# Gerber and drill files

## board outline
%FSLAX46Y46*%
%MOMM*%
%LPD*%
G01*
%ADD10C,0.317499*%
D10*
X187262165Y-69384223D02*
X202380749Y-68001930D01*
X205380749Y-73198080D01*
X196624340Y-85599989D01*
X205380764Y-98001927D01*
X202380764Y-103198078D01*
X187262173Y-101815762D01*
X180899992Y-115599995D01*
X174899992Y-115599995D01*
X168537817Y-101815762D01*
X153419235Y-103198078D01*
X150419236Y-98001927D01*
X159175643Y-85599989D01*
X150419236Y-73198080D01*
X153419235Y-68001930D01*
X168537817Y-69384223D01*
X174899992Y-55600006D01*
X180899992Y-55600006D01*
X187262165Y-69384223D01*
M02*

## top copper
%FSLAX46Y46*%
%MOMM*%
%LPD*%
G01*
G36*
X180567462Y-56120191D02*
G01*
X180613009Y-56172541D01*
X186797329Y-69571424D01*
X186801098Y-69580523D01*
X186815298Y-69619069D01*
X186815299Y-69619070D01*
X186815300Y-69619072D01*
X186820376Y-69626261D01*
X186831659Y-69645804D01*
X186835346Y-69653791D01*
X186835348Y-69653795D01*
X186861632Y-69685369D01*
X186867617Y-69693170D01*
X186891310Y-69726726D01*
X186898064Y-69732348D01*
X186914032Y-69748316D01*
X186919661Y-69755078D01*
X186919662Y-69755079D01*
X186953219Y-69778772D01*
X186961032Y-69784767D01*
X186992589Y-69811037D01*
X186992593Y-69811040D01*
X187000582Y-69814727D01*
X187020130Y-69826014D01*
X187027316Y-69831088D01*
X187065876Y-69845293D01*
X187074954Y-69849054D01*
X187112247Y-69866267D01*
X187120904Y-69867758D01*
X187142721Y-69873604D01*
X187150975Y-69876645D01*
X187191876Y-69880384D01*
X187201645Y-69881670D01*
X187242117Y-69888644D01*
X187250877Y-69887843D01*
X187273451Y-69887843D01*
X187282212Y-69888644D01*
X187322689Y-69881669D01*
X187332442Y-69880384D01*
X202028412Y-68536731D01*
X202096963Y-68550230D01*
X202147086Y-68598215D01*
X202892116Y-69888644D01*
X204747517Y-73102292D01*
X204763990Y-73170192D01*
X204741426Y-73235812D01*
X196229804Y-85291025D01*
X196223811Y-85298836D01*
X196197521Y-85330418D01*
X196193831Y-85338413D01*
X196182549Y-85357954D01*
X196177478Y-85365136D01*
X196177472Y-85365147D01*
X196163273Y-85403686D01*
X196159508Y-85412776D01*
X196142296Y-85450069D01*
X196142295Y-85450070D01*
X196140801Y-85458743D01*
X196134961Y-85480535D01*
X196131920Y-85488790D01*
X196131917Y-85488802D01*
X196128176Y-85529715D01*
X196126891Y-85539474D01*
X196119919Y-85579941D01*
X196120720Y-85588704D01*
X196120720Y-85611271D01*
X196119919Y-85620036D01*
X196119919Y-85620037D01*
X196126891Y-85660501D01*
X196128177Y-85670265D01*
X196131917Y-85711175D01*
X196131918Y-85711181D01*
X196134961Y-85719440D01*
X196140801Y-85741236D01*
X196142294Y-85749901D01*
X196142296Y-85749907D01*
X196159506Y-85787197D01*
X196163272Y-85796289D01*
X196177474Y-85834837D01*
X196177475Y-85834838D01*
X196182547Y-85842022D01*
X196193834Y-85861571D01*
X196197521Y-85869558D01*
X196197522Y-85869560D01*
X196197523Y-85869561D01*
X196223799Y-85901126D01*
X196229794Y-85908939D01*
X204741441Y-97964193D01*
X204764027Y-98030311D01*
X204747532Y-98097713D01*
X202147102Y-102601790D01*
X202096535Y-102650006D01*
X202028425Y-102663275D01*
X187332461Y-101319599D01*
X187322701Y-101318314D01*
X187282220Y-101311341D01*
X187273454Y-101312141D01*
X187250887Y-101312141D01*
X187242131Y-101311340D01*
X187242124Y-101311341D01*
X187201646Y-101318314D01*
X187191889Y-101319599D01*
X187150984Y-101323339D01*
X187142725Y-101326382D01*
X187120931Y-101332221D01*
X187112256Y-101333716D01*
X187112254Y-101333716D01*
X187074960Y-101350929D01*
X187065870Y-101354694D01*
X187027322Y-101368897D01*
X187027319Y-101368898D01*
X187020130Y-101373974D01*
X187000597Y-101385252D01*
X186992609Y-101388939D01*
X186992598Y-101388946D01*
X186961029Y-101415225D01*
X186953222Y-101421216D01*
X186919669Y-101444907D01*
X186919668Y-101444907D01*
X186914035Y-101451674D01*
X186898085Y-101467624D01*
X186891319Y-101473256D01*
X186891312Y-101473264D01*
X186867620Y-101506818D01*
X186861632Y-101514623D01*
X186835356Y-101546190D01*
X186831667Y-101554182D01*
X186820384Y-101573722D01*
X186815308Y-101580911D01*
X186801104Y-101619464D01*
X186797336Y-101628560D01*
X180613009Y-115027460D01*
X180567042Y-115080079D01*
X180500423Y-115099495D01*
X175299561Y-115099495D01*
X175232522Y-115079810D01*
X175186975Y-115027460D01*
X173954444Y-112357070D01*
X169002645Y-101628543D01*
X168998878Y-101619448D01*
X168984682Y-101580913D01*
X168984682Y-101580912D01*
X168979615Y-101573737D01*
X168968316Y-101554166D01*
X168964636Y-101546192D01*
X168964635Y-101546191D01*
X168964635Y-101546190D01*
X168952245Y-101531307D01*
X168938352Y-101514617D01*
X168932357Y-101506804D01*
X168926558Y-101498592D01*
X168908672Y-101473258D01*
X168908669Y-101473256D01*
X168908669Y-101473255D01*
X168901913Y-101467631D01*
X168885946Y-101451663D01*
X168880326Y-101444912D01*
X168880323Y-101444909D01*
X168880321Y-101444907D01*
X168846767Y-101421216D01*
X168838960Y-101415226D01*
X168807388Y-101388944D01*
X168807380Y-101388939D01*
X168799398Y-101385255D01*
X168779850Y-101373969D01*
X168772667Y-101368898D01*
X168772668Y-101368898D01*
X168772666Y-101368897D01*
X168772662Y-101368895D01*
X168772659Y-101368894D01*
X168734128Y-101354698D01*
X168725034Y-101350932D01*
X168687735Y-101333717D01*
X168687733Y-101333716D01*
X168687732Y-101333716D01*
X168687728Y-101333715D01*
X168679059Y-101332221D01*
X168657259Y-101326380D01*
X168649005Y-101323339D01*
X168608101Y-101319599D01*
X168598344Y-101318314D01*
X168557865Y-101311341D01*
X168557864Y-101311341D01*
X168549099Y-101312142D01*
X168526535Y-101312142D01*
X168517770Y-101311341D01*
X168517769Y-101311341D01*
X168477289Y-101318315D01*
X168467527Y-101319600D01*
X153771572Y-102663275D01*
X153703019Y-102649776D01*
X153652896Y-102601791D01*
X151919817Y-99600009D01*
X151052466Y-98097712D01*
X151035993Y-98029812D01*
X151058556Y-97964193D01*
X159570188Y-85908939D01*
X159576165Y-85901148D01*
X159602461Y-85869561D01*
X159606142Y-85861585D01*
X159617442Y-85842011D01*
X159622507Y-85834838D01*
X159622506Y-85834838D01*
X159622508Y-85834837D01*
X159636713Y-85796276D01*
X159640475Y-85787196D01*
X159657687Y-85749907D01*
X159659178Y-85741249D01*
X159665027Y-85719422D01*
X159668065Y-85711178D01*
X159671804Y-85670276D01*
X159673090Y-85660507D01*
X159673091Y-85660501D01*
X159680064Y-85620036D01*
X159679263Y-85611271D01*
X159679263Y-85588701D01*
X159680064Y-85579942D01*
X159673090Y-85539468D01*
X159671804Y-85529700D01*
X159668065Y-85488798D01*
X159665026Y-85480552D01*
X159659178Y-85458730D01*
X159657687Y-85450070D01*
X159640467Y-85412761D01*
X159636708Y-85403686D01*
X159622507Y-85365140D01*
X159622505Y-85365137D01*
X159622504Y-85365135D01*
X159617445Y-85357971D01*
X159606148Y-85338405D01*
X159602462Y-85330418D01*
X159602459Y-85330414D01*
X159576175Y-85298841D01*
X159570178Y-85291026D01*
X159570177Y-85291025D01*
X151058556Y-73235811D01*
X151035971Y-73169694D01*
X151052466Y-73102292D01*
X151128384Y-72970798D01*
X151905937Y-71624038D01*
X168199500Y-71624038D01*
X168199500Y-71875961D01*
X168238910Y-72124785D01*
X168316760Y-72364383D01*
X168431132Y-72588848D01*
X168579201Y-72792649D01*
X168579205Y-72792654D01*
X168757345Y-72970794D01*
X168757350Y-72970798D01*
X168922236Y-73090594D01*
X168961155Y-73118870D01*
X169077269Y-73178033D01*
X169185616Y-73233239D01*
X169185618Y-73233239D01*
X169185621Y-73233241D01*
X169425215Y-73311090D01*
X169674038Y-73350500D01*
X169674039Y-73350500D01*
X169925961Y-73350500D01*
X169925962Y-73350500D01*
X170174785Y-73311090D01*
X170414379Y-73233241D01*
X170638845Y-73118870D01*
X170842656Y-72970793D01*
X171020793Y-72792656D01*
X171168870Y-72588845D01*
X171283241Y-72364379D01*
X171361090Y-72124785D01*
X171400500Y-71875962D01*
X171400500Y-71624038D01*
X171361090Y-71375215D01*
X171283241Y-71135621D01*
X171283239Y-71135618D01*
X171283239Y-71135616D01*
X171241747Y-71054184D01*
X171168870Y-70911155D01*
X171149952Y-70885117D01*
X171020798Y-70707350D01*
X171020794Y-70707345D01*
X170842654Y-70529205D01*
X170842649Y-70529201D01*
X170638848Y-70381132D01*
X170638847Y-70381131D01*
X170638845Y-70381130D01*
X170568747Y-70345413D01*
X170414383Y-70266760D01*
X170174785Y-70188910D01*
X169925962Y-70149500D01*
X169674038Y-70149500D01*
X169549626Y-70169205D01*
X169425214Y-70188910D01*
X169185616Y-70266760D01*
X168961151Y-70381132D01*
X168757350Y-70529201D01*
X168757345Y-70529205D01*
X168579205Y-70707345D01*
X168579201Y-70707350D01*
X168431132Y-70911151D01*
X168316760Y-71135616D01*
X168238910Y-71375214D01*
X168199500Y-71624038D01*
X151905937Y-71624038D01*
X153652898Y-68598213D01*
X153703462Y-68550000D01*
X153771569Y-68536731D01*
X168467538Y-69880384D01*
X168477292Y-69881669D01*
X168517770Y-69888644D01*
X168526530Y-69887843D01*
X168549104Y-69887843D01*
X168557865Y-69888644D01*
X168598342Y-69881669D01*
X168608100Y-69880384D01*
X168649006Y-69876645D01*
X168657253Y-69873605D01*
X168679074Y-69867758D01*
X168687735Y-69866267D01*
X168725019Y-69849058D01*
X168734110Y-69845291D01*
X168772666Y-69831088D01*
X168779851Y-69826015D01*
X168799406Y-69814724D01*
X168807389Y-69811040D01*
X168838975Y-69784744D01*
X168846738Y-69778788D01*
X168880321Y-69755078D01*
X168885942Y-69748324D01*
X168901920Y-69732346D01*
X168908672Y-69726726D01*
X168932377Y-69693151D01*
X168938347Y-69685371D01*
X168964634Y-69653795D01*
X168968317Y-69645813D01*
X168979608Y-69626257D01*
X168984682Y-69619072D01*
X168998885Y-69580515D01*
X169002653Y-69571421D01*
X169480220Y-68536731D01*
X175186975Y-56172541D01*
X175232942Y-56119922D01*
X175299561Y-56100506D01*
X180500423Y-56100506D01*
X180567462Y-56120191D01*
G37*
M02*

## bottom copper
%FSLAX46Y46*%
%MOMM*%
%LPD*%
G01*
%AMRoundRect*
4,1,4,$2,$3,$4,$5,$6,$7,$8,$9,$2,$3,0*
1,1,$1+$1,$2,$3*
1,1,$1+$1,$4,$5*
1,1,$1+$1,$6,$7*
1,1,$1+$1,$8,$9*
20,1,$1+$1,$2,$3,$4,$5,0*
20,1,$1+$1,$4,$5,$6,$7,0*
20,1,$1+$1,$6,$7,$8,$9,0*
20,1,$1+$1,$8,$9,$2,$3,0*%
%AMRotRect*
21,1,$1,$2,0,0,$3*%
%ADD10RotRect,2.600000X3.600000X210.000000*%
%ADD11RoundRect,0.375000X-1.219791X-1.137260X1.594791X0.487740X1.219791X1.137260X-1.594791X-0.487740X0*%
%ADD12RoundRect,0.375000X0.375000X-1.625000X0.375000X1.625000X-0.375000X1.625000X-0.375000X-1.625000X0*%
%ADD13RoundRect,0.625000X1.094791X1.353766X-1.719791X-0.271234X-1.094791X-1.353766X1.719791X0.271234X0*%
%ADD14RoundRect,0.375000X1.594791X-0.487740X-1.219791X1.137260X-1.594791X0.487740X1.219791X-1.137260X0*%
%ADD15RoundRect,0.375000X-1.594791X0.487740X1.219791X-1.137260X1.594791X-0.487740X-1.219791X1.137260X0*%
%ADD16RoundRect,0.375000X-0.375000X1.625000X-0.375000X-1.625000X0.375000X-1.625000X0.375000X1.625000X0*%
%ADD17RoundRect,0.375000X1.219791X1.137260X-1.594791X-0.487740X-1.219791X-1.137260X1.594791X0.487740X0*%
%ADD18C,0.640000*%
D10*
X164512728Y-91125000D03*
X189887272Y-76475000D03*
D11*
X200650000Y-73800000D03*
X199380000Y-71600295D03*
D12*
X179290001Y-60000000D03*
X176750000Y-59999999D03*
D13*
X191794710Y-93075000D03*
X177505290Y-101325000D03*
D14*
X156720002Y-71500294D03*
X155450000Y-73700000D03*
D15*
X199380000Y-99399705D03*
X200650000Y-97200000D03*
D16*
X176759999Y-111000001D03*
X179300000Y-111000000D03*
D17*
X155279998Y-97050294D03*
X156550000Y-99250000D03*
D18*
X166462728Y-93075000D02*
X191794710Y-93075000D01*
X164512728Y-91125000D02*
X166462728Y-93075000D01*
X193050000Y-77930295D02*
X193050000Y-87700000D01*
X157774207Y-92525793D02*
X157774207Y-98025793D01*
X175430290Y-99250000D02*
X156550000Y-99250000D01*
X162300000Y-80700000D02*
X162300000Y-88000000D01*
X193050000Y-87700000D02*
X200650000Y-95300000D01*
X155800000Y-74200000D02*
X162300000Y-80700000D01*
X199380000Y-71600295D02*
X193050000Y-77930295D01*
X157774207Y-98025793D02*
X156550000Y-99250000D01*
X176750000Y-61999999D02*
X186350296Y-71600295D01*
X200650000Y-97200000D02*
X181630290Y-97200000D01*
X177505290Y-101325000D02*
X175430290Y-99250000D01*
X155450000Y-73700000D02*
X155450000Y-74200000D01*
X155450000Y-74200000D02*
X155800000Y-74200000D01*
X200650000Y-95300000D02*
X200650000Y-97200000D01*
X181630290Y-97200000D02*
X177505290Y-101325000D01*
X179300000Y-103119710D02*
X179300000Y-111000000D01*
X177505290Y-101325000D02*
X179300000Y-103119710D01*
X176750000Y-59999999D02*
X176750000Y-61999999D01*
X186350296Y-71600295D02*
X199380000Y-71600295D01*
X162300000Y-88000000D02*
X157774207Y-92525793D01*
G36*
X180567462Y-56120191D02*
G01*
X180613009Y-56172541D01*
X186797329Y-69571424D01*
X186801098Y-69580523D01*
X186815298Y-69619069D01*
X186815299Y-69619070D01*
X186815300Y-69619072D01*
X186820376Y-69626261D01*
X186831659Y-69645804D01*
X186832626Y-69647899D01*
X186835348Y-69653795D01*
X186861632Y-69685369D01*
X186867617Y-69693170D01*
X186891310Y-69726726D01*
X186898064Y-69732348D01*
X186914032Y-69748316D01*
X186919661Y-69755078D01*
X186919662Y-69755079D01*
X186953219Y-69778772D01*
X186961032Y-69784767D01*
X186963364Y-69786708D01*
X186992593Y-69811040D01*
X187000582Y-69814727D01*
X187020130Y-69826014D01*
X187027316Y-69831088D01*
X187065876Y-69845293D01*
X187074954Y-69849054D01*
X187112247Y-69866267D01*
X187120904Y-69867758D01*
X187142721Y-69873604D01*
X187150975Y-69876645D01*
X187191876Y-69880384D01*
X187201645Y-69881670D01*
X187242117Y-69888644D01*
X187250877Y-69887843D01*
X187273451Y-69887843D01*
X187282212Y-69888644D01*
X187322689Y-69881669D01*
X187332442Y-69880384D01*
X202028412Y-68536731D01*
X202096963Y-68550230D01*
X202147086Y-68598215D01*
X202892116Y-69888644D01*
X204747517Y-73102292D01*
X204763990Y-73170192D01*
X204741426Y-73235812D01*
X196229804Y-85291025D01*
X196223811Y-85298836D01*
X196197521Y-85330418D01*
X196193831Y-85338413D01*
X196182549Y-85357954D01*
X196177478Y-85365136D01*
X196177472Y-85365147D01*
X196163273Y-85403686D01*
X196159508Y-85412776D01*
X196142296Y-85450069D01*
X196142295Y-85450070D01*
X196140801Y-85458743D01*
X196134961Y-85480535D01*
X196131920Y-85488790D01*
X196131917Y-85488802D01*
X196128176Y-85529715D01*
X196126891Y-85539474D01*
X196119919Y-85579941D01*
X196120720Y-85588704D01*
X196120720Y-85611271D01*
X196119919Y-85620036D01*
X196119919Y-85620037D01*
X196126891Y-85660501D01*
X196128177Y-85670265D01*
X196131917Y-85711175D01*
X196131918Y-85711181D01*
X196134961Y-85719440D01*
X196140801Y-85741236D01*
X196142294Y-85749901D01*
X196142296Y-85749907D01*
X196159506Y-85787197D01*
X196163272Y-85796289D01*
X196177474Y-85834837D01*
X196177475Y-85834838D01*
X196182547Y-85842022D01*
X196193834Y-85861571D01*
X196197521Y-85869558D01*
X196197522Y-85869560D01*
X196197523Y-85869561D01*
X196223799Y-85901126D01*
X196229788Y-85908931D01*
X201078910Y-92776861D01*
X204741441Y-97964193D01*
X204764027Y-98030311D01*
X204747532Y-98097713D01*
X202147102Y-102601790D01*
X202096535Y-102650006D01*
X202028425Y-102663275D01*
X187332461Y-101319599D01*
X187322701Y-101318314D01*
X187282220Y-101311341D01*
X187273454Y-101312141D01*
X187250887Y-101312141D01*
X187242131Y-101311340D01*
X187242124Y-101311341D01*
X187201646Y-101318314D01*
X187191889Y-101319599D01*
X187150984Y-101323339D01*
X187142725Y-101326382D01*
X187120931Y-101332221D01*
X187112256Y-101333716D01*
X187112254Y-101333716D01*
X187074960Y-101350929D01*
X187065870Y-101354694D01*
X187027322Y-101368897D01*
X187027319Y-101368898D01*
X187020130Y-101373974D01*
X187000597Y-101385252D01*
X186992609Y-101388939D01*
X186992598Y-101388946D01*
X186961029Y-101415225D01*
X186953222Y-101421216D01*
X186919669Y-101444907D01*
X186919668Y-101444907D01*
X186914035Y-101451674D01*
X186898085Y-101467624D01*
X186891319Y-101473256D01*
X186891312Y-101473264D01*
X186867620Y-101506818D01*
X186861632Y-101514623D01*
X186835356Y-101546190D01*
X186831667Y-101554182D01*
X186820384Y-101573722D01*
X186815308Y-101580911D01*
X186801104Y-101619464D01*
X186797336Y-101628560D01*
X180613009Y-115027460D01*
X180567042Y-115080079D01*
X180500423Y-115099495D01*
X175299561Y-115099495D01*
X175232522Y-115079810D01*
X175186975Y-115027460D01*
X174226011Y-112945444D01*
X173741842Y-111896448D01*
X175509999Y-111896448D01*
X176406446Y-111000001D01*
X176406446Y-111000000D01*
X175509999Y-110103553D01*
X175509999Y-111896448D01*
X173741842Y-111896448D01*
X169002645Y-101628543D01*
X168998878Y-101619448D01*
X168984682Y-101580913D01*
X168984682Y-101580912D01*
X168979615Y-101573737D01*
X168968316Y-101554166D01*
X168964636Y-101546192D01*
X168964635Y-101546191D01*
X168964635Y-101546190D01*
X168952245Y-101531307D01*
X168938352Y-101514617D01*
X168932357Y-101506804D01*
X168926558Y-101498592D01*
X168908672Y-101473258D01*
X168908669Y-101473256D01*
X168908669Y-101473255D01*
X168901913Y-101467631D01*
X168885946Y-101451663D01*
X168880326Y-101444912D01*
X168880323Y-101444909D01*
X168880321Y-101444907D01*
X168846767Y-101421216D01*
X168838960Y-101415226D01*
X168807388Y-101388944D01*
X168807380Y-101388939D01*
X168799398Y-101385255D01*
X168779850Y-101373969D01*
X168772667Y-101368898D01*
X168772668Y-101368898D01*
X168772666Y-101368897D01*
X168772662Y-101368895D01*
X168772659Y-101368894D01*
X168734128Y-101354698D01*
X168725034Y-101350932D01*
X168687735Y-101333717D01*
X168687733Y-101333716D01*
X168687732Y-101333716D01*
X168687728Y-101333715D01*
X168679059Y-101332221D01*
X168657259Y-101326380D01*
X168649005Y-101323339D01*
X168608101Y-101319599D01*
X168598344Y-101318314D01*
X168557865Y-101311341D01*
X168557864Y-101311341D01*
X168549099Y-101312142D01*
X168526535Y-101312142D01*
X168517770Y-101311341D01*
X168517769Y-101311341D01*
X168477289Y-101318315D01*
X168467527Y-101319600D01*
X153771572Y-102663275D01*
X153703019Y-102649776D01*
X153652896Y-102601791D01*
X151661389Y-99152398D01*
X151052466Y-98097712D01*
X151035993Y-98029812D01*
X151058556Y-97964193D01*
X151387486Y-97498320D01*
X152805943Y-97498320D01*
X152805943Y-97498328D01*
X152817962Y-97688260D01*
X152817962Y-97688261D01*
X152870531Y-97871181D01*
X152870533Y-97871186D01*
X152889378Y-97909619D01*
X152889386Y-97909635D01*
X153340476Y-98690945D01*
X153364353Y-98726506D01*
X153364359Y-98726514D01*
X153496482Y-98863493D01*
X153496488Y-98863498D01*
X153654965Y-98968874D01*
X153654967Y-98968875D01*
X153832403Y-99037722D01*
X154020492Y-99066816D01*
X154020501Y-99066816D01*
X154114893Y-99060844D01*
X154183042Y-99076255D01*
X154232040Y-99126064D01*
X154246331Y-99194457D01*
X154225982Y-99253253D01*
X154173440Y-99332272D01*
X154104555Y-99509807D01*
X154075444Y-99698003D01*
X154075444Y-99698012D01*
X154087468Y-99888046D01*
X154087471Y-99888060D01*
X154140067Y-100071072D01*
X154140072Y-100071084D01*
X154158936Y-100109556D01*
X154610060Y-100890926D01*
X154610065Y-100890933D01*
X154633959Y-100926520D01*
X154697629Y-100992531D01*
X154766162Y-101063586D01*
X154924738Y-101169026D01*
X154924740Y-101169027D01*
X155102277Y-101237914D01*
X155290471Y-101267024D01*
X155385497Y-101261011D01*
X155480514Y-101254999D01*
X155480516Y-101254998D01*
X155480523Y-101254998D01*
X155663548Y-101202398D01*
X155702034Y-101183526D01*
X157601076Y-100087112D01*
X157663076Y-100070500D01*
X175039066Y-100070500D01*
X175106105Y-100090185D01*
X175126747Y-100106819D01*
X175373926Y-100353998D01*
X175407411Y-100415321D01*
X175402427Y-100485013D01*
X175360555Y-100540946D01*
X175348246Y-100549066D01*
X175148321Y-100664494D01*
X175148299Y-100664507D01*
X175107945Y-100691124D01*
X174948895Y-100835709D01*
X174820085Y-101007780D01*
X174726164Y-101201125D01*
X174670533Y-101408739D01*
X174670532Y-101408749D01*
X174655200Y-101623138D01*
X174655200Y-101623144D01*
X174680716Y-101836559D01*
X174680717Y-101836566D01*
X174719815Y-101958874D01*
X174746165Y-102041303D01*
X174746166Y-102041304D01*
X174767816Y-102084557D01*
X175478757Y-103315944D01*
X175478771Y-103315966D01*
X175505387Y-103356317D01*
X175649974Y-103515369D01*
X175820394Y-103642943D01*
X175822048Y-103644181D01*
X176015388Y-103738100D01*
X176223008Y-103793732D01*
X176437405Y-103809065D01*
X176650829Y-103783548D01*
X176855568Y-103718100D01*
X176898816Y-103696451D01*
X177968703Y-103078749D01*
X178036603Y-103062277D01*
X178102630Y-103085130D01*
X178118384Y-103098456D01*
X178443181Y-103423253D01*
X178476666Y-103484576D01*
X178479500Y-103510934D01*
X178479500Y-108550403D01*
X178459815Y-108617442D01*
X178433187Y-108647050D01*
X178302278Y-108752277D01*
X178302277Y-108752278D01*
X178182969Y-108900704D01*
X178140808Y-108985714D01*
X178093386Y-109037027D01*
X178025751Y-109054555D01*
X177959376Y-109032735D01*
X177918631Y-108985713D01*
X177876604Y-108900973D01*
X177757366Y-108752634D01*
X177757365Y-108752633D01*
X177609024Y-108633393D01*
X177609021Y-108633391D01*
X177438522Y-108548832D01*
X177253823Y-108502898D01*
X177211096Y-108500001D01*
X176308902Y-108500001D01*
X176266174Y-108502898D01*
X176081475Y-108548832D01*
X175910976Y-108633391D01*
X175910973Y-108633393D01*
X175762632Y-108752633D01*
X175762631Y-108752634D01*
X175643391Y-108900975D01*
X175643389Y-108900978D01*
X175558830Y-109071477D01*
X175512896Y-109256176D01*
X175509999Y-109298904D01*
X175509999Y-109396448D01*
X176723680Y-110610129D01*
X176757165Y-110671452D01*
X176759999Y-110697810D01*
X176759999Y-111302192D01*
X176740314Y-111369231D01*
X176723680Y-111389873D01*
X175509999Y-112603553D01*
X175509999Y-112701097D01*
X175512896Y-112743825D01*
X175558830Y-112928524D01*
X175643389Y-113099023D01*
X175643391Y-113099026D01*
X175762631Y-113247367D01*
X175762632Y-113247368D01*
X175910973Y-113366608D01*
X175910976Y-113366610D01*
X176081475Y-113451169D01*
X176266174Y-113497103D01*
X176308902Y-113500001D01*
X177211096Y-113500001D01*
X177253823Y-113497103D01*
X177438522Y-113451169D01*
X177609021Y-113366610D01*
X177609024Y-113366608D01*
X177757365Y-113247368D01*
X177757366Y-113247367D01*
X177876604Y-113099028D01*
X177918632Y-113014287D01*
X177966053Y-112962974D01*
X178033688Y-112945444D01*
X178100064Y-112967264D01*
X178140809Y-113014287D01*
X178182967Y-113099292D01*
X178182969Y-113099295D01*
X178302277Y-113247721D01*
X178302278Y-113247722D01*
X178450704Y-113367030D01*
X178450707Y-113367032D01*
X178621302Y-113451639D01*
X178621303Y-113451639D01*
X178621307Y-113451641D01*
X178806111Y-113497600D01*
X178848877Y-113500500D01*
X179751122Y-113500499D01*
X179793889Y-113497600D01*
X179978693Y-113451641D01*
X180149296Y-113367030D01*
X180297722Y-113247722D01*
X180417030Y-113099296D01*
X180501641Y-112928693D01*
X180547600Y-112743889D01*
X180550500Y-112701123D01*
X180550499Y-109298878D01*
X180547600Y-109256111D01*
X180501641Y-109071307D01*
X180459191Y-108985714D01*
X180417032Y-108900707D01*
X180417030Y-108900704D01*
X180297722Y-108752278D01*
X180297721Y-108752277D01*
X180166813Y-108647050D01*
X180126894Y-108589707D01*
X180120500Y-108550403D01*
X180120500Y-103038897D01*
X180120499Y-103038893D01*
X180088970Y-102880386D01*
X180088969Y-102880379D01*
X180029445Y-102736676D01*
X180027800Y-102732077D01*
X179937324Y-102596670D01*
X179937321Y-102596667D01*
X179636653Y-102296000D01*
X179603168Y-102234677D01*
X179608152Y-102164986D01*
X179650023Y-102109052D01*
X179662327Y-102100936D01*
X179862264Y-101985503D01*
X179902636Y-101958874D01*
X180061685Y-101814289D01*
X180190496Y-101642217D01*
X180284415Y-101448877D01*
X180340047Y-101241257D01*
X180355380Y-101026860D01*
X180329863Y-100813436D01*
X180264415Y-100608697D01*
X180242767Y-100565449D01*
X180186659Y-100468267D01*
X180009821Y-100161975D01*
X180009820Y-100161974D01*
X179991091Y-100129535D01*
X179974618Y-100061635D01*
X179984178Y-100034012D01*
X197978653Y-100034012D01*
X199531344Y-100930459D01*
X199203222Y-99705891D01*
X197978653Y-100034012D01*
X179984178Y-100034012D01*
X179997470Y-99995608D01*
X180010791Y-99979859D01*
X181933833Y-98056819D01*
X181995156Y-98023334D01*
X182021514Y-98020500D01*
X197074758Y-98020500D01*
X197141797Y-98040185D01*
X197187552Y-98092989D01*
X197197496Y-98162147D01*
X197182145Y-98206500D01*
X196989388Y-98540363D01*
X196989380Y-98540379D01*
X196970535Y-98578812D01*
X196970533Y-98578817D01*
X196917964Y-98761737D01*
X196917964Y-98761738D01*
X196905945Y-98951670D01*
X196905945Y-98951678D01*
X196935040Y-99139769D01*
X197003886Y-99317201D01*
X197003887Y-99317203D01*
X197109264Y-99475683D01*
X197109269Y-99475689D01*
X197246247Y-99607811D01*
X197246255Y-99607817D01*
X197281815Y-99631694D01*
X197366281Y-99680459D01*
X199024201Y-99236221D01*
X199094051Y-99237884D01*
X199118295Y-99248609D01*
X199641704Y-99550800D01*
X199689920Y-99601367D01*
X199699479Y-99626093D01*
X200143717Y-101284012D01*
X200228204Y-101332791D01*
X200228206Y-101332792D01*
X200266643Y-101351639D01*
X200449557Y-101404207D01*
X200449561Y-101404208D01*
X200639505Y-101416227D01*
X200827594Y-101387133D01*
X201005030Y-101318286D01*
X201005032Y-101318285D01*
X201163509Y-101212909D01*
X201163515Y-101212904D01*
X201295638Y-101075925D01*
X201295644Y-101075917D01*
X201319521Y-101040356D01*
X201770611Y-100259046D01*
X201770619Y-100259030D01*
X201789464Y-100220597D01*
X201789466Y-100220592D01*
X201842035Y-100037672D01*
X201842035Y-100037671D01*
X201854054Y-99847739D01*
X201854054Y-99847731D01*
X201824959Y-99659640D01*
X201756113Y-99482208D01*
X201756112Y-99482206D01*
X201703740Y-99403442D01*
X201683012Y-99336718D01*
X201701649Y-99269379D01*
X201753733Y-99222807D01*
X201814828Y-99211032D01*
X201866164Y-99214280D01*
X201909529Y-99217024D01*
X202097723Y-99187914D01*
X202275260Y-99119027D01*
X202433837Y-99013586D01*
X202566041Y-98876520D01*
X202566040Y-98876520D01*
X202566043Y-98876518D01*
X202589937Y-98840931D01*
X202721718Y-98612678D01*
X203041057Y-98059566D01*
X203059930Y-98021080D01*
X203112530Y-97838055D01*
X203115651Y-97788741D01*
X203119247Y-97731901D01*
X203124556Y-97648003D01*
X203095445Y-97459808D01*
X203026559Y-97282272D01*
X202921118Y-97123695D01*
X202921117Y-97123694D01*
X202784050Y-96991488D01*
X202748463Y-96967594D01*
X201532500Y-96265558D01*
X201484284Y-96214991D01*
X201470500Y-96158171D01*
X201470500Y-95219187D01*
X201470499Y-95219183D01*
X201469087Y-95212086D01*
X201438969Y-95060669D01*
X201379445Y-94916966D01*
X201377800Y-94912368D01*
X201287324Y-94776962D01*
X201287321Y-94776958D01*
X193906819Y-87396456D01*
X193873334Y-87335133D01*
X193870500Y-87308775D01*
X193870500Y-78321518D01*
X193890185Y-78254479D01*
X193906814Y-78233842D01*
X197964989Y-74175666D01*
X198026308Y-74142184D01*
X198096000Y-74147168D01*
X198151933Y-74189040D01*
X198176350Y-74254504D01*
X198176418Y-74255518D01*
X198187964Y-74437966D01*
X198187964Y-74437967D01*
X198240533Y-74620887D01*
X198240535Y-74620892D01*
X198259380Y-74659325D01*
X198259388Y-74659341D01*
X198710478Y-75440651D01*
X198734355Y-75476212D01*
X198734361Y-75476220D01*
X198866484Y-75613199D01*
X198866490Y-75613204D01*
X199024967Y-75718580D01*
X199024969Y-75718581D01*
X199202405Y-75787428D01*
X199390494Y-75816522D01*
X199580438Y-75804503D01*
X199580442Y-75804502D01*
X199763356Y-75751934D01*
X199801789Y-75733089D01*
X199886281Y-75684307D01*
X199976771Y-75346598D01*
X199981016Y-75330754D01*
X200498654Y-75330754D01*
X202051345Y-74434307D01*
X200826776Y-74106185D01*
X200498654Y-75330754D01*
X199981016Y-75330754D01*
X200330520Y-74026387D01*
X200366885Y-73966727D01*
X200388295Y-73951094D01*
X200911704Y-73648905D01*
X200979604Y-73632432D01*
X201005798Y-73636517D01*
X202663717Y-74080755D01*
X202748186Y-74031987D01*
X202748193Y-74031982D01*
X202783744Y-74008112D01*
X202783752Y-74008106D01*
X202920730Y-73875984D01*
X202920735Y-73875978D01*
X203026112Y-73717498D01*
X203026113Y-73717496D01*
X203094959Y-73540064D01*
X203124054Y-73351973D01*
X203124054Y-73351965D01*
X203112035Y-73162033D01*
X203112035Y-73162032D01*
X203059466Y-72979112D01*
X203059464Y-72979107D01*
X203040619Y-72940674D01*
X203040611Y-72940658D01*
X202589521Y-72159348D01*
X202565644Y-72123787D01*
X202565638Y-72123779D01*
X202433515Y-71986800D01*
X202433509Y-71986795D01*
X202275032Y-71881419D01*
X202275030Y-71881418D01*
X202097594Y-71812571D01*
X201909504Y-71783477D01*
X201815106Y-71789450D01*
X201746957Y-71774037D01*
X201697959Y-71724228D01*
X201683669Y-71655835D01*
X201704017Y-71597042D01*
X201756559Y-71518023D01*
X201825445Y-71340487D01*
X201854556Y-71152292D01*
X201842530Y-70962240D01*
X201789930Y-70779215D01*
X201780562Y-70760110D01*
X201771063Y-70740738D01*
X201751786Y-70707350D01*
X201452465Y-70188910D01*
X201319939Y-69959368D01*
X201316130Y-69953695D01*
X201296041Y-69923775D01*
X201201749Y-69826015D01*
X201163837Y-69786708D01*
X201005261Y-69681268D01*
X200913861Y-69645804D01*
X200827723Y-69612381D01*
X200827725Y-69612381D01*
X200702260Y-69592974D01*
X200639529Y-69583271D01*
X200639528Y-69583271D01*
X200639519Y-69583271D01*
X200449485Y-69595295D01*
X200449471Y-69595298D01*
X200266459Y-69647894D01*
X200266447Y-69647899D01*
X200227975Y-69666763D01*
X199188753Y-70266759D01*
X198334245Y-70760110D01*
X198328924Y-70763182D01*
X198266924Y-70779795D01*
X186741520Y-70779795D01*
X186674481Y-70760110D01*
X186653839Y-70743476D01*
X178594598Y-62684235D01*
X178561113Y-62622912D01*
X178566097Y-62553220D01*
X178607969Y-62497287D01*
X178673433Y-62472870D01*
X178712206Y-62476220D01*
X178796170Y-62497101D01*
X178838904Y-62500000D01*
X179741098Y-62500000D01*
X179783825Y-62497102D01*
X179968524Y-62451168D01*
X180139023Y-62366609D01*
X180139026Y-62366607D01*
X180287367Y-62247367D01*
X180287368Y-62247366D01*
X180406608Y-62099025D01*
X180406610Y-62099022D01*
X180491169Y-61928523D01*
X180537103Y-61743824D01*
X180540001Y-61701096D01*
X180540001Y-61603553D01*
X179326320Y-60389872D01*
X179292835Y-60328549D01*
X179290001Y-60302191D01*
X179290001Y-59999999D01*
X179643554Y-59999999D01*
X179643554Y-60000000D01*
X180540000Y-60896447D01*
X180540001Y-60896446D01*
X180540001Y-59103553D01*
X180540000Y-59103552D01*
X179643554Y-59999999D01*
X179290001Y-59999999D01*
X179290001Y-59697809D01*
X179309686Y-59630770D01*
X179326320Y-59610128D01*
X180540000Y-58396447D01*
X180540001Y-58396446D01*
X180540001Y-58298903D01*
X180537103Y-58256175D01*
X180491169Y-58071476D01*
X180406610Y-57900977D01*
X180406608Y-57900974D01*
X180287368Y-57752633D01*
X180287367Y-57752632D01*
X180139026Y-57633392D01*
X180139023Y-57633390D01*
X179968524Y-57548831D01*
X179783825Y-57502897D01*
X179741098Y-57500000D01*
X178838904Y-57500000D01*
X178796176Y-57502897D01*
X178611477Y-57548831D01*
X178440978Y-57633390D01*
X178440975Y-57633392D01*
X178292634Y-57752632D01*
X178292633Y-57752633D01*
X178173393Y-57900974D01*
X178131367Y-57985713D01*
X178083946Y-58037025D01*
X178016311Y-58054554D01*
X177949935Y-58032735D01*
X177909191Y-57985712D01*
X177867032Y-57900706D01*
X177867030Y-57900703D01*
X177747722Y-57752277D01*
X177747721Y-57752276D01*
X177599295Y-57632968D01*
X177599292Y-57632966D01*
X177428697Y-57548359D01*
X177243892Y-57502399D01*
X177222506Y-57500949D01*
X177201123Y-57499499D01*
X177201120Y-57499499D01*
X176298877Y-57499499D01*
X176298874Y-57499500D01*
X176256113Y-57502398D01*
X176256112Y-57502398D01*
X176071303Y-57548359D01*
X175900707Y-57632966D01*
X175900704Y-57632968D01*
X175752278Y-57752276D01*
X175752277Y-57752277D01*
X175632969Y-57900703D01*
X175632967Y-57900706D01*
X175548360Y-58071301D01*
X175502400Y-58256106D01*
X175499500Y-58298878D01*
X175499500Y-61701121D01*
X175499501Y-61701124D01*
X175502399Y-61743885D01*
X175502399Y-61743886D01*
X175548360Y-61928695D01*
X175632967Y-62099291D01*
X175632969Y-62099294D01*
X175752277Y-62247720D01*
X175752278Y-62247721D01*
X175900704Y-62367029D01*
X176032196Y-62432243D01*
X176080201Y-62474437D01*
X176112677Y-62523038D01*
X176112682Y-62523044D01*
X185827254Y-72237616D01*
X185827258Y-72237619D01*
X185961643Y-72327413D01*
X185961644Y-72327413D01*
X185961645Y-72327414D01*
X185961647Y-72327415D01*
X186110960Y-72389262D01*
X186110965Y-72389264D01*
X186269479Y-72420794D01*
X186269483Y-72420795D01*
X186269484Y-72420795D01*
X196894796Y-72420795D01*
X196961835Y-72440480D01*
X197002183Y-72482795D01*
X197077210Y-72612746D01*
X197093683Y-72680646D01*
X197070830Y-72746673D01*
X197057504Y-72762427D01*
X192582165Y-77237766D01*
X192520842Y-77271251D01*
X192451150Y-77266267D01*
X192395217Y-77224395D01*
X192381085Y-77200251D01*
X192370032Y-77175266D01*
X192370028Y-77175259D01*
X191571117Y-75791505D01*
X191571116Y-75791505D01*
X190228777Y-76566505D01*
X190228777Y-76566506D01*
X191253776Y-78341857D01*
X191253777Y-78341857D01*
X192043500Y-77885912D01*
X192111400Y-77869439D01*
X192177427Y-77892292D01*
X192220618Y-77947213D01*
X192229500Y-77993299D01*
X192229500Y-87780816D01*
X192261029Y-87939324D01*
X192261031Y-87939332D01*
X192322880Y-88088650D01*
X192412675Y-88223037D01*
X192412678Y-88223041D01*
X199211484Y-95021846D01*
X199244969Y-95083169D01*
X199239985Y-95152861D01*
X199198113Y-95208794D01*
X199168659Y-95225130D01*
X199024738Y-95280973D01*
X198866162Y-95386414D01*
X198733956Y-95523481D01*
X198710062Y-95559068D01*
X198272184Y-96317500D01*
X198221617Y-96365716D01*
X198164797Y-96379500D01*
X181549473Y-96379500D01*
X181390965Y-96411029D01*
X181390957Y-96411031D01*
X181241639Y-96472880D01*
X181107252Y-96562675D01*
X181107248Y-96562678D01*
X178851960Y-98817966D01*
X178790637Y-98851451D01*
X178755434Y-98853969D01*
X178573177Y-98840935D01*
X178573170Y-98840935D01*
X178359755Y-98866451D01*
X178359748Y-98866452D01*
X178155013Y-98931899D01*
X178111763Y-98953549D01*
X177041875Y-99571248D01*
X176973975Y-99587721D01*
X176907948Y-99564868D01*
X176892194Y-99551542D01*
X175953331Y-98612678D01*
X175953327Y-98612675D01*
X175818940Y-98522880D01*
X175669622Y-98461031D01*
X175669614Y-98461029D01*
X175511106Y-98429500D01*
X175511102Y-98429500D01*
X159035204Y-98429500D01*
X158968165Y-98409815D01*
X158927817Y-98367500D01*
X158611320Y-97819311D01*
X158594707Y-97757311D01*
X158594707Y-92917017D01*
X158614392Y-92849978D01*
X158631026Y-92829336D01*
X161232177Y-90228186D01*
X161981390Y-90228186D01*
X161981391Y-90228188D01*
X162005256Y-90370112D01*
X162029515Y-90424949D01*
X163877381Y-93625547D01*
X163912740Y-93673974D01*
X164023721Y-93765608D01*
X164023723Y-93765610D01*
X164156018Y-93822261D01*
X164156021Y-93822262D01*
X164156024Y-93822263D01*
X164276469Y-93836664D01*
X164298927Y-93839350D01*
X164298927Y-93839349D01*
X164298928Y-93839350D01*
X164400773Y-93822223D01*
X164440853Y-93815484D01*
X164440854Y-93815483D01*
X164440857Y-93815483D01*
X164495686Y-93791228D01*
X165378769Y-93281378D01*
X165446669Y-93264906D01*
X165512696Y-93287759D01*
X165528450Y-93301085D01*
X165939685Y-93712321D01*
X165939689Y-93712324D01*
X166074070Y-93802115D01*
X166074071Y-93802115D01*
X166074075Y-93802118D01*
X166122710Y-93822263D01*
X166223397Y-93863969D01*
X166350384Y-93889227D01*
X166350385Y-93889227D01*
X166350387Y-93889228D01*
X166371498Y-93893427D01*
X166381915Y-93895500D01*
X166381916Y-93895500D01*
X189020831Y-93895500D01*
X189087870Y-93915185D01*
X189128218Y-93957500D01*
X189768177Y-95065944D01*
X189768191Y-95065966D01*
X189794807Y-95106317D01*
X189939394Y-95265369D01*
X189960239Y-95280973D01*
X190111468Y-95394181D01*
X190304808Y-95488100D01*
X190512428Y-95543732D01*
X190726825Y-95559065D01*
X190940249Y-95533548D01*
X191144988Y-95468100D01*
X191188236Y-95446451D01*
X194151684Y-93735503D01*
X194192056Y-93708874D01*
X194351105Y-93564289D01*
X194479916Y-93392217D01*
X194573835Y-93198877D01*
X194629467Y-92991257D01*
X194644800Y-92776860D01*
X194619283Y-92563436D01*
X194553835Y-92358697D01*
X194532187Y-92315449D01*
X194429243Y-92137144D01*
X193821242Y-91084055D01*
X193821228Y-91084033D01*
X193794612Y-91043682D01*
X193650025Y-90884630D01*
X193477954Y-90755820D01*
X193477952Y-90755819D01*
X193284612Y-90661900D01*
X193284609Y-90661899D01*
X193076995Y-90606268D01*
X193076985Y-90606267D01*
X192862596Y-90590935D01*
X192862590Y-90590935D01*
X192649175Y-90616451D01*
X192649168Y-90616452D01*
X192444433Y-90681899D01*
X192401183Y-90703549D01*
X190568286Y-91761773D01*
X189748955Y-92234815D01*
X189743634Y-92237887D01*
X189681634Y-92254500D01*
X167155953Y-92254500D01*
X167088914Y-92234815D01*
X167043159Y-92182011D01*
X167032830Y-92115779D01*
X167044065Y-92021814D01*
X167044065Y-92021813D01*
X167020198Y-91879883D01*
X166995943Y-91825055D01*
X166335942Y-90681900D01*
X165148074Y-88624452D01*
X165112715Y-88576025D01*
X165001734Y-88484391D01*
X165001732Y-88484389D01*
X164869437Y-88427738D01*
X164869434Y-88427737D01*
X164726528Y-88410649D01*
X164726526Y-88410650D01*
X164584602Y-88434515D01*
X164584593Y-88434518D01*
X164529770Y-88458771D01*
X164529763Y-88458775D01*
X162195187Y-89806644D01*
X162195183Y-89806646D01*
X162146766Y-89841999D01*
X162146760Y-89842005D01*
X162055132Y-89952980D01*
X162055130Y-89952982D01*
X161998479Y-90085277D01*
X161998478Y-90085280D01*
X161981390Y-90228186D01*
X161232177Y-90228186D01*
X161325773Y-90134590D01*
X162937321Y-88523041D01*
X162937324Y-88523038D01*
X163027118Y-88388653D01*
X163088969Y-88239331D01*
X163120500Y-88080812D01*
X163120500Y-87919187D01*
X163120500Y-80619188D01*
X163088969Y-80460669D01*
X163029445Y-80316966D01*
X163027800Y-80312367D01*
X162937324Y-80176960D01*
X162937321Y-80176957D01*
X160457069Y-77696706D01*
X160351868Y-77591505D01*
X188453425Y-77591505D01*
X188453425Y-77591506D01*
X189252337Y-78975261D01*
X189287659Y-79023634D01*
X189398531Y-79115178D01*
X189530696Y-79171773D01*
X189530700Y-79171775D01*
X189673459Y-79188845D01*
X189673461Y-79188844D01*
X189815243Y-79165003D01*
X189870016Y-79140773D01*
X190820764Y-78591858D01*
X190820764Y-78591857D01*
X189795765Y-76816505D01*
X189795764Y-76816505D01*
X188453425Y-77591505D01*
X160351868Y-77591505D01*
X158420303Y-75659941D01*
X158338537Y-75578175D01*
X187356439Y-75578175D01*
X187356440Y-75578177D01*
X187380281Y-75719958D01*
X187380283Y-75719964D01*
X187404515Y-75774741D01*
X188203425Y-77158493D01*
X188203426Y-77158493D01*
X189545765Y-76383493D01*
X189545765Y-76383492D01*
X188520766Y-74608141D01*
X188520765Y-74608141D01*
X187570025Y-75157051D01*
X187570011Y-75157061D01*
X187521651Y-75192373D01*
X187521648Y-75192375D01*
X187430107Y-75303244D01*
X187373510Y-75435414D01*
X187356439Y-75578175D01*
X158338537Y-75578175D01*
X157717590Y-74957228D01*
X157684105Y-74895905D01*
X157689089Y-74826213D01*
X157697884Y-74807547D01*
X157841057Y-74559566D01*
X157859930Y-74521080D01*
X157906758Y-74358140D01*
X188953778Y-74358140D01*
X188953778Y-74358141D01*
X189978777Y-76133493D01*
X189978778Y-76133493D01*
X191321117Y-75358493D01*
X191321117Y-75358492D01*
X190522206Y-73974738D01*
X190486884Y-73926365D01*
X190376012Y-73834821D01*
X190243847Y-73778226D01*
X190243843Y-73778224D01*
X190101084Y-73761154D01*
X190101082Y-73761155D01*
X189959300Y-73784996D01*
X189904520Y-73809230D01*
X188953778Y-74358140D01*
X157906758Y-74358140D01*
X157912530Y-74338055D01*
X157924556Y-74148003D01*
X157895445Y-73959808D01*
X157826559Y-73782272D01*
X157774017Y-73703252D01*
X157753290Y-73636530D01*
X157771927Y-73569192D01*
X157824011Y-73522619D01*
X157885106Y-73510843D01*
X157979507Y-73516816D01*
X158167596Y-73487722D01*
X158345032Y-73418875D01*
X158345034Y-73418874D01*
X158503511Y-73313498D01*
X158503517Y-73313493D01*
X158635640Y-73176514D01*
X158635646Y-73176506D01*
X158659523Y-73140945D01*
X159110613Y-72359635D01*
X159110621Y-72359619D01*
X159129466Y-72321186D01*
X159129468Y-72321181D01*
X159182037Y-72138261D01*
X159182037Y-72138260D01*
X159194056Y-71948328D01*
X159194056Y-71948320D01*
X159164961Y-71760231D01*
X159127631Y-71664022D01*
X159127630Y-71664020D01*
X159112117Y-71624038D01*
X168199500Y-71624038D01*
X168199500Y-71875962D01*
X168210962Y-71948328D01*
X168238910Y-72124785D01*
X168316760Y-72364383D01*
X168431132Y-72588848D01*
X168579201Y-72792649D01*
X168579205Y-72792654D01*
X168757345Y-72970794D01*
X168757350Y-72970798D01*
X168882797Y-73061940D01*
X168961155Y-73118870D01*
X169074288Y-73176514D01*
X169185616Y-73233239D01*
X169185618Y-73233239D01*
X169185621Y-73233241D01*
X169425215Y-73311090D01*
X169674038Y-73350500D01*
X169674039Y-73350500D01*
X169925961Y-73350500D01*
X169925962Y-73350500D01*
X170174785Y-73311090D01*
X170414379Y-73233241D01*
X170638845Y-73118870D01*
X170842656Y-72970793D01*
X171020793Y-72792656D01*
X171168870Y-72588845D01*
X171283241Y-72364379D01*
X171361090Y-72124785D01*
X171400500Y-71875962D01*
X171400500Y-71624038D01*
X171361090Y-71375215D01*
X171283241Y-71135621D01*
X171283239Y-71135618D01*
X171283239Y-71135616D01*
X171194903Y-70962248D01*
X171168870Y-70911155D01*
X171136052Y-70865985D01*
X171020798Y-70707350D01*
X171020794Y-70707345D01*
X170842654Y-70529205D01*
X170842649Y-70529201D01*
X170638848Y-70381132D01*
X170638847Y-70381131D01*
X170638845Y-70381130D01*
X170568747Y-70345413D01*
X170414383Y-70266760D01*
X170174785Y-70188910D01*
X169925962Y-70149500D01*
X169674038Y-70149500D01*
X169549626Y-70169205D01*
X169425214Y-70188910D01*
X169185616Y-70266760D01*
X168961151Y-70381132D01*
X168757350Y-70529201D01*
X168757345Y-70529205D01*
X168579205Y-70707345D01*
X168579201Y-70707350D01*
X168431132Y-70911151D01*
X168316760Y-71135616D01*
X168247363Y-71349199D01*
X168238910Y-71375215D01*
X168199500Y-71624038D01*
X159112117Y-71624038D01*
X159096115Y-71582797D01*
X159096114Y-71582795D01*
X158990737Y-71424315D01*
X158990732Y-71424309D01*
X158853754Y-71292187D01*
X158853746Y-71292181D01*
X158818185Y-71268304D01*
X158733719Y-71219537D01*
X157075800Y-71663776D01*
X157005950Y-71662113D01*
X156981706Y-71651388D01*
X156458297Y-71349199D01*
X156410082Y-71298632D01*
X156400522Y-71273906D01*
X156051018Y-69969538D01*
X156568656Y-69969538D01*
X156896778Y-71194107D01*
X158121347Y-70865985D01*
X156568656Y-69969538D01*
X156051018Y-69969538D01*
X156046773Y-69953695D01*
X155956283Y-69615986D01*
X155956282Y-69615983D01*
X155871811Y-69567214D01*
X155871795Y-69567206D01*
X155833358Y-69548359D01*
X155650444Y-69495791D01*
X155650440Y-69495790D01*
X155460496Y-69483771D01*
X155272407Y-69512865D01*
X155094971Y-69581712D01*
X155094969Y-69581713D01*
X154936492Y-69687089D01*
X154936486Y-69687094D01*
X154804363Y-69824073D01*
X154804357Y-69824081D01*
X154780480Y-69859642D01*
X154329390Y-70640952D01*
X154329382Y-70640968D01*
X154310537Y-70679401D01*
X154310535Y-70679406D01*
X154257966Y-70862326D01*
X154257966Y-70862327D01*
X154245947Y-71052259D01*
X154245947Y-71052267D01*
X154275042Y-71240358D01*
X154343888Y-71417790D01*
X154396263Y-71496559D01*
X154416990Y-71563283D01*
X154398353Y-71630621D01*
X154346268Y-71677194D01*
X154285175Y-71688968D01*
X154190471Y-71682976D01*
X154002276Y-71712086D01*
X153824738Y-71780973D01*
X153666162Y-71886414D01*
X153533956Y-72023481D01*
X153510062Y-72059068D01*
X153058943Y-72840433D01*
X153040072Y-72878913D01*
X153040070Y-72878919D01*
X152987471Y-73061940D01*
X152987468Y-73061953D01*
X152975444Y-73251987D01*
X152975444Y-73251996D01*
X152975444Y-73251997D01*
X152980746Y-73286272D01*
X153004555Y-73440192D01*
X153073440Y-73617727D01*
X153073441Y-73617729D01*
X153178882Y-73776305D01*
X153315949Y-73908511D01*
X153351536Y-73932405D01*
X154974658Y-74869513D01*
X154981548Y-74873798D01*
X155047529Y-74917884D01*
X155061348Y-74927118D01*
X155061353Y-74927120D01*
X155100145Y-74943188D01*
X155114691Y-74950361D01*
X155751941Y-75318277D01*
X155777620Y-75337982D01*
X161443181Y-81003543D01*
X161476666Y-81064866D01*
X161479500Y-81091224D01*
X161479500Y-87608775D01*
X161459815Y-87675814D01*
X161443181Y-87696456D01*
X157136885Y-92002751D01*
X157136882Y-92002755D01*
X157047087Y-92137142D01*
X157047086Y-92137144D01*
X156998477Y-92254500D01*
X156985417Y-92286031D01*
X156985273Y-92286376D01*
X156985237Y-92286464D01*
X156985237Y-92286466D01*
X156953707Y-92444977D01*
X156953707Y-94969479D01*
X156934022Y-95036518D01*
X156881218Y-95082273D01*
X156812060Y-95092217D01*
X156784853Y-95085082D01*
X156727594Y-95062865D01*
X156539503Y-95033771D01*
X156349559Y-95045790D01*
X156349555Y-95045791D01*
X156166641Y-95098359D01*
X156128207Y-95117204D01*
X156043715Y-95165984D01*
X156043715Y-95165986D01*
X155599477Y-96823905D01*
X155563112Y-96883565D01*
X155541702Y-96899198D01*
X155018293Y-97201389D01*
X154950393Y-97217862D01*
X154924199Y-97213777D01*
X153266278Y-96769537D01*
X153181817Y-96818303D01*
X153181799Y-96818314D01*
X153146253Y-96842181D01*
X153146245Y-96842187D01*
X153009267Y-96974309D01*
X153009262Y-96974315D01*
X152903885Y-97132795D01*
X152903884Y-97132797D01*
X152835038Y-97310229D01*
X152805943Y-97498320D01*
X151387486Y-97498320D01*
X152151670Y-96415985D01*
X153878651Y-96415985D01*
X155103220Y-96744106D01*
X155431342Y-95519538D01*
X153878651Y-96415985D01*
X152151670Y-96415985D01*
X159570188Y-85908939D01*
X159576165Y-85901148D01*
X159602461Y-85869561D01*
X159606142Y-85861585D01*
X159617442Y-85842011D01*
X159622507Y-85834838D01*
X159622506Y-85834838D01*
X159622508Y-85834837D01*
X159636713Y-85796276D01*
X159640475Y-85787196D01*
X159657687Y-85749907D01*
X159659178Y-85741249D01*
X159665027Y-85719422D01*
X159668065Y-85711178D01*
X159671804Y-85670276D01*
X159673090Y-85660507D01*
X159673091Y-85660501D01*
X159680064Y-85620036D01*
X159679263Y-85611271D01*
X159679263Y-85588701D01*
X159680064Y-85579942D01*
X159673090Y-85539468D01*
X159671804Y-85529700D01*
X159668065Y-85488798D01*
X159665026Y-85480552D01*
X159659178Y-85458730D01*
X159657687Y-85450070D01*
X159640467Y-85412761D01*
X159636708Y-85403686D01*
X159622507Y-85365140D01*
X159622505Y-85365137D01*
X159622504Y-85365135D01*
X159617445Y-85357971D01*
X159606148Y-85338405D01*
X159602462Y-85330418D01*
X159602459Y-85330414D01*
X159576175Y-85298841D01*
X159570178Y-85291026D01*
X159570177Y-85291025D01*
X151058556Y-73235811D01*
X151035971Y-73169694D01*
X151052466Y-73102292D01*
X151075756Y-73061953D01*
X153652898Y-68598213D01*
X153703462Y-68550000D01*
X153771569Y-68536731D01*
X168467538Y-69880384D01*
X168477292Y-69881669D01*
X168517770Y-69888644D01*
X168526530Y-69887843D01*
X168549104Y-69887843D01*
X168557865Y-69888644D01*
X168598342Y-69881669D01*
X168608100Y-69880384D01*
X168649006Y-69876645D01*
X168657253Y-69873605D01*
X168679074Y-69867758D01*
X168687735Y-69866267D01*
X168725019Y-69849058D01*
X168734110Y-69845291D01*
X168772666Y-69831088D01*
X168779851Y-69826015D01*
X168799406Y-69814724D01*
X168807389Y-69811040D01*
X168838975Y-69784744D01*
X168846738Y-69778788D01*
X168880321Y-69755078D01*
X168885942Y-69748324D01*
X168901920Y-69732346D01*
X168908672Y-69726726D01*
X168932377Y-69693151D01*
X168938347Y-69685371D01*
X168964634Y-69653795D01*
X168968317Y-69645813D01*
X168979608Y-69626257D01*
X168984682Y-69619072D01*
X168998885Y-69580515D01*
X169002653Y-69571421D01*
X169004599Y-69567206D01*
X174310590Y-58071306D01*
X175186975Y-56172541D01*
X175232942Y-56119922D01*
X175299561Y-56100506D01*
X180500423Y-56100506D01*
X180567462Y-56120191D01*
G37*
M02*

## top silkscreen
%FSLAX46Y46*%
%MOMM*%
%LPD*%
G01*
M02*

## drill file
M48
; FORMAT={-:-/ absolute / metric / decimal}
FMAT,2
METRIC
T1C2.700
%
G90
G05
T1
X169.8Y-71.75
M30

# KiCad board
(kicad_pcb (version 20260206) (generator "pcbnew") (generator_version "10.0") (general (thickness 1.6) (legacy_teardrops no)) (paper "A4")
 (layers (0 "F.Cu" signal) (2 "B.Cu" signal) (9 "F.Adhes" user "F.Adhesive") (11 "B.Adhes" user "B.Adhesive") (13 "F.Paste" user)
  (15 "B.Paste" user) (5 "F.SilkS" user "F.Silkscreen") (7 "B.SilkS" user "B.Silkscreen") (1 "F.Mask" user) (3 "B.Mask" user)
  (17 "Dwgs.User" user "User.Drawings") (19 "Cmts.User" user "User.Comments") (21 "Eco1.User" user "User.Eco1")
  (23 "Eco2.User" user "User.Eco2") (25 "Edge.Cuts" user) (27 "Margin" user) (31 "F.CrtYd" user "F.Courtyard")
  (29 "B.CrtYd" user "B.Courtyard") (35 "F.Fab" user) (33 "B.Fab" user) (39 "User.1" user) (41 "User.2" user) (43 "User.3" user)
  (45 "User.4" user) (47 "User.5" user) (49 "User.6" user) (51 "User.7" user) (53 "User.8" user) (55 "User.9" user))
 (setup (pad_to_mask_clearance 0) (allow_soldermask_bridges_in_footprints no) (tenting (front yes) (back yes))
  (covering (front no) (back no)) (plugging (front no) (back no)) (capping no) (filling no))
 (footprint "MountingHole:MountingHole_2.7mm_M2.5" (layer "F.Cu") (at 169.8 71.75)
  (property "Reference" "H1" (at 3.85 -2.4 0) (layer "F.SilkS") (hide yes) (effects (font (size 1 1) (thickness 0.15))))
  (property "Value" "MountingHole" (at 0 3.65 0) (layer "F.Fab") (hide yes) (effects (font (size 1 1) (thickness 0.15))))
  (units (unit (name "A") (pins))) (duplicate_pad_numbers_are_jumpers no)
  (pad "" np_thru_hole circle (at 0 0) (size 2.7 2.7) (drill 2.7) (layers "*.Cu" "*.Mask")))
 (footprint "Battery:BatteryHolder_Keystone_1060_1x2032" (layer "B.Cu") (at 177.2 83.8 30)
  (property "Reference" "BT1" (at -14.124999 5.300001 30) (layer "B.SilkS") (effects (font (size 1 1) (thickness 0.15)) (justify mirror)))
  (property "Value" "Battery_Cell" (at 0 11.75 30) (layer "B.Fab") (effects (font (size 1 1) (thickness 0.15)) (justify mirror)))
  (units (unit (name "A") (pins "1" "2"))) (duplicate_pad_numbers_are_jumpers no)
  (pad "1" smd rect (at -14.65 0 210) (size 2.6 3.6) (layers "B.Cu" "B.Mask" "B.Paste") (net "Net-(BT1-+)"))
  (pad "2" smd rect (at 14.65 0 210) (size 2.6 3.6) (layers "B.Cu" "B.Mask" "B.Paste") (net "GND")))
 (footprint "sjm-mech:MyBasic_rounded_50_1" (layer "B.Cu") (at 160.75 74.75 -120)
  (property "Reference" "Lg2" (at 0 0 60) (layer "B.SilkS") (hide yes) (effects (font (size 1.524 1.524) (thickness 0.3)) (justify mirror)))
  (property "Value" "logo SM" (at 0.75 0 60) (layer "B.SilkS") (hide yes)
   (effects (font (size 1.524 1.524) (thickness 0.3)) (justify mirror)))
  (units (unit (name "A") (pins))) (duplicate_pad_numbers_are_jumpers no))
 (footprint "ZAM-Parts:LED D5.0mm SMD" (layer "B.Cu") (at 200.65 73.8 30)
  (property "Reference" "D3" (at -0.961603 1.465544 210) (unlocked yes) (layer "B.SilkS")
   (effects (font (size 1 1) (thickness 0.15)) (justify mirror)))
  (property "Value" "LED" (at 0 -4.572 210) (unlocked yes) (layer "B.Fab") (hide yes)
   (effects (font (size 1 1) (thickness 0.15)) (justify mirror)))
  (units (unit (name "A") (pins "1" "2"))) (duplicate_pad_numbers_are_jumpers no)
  (pad "1" smd roundrect (at 0 0 30) (size 4 1.5) (layers "B.Cu" "B.Mask" "B.Paste") (roundrect_rratio 0.25) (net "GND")
   (thermal_bridge_angle 45))
  (pad "2" smd roundrect (at 0 -2.54 30) (size 4 1.5) (layers "B.Cu" "B.Mask" "B.Paste") (roundrect_rratio 0.25) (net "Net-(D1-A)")
   (thermal_bridge_angle 45)))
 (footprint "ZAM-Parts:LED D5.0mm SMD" (layer "B.Cu") (at 179.290001 60 90)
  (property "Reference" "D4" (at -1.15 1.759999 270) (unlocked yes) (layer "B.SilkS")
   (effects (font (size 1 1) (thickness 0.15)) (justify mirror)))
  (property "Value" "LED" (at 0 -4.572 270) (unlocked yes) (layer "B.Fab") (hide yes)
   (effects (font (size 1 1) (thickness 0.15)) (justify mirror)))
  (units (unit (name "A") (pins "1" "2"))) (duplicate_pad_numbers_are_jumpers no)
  (pad "1" smd roundrect (at 0 0 90) (size 4 1.5) (layers "B.Cu" "B.Mask" "B.Paste") (roundrect_rratio 0.25) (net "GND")
   (thermal_bridge_angle 45))
  (pad "2" smd roundrect (at 0.000001 -2.540001 90) (size 4 1.5) (layers "B.Cu" "B.Mask" "B.Paste") (roundrect_rratio 0.25)
   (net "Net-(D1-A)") (thermal_bridge_angle 45)))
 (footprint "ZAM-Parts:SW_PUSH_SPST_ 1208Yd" (layer "B.Cu") (at 184.65 97.2 -150)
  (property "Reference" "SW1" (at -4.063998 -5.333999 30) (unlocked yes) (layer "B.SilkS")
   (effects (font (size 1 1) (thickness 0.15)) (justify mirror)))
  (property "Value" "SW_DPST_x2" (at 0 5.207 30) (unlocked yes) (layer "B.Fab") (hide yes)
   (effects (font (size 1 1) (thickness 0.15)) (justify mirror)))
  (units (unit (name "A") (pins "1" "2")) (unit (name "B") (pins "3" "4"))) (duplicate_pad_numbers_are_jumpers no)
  (pad "1" smd roundrect (at -8.25 0 210) (size 4.5 2.5) (layers "B.Cu" "B.Mask" "B.Paste") (roundrect_rratio 0.25) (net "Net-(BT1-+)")
   (thermal_bridge_angle 45))
  (pad "2" smd roundrect (at 8.25 0 210) (size 4.5 2.5) (layers "B.Cu" "B.Mask" "B.Paste") (roundrect_rratio 0.25) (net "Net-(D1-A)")
   (thermal_bridge_angle 45)))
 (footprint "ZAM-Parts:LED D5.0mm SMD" (layer "B.Cu") (at 156.720002 71.500294 150)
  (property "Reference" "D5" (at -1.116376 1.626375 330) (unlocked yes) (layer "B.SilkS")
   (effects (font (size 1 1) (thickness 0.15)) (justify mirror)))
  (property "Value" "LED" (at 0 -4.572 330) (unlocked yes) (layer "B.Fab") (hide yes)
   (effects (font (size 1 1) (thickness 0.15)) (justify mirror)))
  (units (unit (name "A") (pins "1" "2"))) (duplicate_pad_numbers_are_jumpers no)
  (pad "1" smd roundrect (at 0 0 150) (size 4 1.5) (layers "B.Cu" "B.Mask" "B.Paste") (roundrect_rratio 0.25) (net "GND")
   (thermal_bridge_angle 45))
  (pad "2" smd roundrect (at 0.000001 -2.540002 150) (size 4 1.5) (layers "B.Cu" "B.Mask" "B.Paste") (roundrect_rratio 0.25)
   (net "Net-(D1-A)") (thermal_bridge_angle 45)))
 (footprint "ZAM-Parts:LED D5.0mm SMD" (layer "B.Cu") (at 199.38 99.399705 -30)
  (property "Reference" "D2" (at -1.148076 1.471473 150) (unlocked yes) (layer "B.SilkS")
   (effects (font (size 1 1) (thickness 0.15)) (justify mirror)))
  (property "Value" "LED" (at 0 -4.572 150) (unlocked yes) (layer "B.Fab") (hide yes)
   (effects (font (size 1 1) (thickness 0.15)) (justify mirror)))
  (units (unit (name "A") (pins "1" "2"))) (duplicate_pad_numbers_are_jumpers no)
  (pad "1" smd roundrect (at 0 0 330) (size 4 1.5) (layers "B.Cu" "B.Mask" "B.Paste") (roundrect_rratio 0.25) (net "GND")
   (thermal_bridge_angle 45))
  (pad "2" smd roundrect (at 0 -2.54 330) (size 4 1.5) (layers "B.Cu" "B.Mask" "B.Paste") (roundrect_rratio 0.25) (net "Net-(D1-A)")
   (thermal_bridge_angle 45)))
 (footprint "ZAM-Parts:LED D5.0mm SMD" (layer "B.Cu") (at 176.759999 111.000001 -90)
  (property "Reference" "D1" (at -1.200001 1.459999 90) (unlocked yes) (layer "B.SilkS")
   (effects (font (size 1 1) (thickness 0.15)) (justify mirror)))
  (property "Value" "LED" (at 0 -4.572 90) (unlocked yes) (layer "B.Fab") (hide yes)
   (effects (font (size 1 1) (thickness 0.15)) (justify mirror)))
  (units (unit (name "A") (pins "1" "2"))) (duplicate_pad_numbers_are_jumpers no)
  (pad "1" smd roundrect (at 0 0 270) (size 4 1.5) (layers "B.Cu" "B.Mask" "B.Paste") (roundrect_rratio 0.25) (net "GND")
   (thermal_bridge_angle 45))
  (pad "2" smd roundrect (at -0.000001 -2.540001 270) (size 4 1.5) (layers "B.Cu" "B.Mask" "B.Paste") (roundrect_rratio 0.25)
   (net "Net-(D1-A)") (thermal_bridge_angle 45)))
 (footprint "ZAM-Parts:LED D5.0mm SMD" (layer "B.Cu") (at 155.279998 97.050294 -150)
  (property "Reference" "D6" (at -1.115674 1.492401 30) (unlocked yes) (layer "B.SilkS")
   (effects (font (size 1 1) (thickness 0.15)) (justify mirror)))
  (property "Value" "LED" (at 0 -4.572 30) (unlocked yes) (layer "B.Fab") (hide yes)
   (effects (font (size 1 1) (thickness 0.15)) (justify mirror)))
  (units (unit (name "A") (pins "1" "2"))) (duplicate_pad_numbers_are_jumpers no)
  (pad "1" smd roundrect (at 0 0 210) (size 4 1.5) (layers "B.Cu" "B.Mask" "B.Paste") (roundrect_rratio 0.25) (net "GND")
   (thermal_bridge_angle 45))
  (pad "2" smd roundrect (at -0.000001 -2.540002 210) (size 4 1.5) (layers "B.Cu" "B.Mask" "B.Paste") (roundrect_rratio 0.25)
   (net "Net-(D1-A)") (thermal_bridge_angle 45)))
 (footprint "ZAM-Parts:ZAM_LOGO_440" (layer "B.Cu") (at 177.887717 65.535372 180)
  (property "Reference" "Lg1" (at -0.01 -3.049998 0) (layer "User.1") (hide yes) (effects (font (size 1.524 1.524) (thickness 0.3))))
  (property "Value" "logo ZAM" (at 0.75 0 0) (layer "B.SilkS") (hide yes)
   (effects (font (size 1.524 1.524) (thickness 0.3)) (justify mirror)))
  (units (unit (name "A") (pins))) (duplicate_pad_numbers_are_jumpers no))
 (gr_poly
  (pts (xy 187.262165 69.384223) (xy 202.380749 68.00193) (xy 205.380749 73.19808) (xy 196.62434 85.599989) (xy 205.380764 98.001927)
   (xy 202.380764 103.198078) (xy 187.262173 101.815762) (xy 180.899992 115.599995) (xy 174.899992 115.599995) (xy 168.537817 101.815762)
   (xy 153.419235 103.198078) (xy 150.419236 98.001927) (xy 159.175643 85.599989) (xy 150.419236 73.19808) (xy 153.419235 68.00193)
   (xy 168.537817 69.384223) (xy 174.899992 55.600006) (xy 180.899992 55.600006))
  (stroke (width 0.317499) (type solid)) (fill no) (layer "Edge.Cuts"))
 (segment (start 166.462728 93.075) (end 191.79471 93.075) (width 0.64) (layer "B.Cu") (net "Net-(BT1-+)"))
 (segment (start 164.512728 91.125) (end 166.462728 93.075) (width 0.64) (layer "B.Cu") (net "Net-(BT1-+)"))
 (segment (start 193.05 77.930295) (end 193.05 87.7) (width 0.64) (layer "B.Cu") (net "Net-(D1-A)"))
 (segment (start 157.774207 92.525793) (end 157.774207 98.025793) (width 0.64) (layer "B.Cu") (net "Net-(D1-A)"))
 (segment (start 175.43029 99.25) (end 156.55 99.25) (width 0.64) (layer "B.Cu") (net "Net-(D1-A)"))
 (segment (start 162.3 80.7) (end 162.3 88) (width 0.64) (layer "B.Cu") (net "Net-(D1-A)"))
 (segment (start 193.05 87.7) (end 200.65 95.3) (width 0.64) (layer "B.Cu") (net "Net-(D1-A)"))
 (segment (start 155.8 74.2) (end 162.3 80.7) (width 0.64) (layer "B.Cu") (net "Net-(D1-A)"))
 (segment (start 199.38 71.600295) (end 193.05 77.930295) (width 0.64) (layer "B.Cu") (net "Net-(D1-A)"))
 (segment (start 157.774207 98.025793) (end 156.55 99.25) (width 0.64) (layer "B.Cu") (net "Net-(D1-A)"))
 (segment (start 176.75 61.999999) (end 186.350296 71.600295) (width 0.64) (layer "B.Cu") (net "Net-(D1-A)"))
 (segment (start 200.65 97.2) (end 181.63029 97.2) (width 0.64) (layer "B.Cu") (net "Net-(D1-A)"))
 (segment (start 177.50529 101.325) (end 175.43029 99.25) (width 0.64) (layer "B.Cu") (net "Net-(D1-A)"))
 (segment (start 155.45 73.7) (end 155.45 74.2) (width 0.64) (layer "B.Cu") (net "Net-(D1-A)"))
 (segment (start 155.45 74.2) (end 155.8 74.2) (width 0.64) (layer "B.Cu") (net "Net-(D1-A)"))
 (segment (start 200.65 95.3) (end 200.65 97.2) (width 0.64) (layer "B.Cu") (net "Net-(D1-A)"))
 (segment (start 181.63029 97.2) (end 177.50529 101.325) (width 0.64) (layer "B.Cu") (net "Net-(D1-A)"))
 (segment (start 179.3 103.11971) (end 179.3 111) (width 0.64) (layer "B.Cu") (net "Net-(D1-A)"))
 (segment (start 177.50529 101.325) (end 179.3 103.11971) (width 0.64) (layer "B.Cu") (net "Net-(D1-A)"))
 (segment (start 176.75 59.999999) (end 176.75 61.999999) (width 0.64) (layer "B.Cu") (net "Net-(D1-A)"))
 (segment (start 186.350296 71.600295) (end 199.38 71.600295) (width 0.64) (layer "B.Cu") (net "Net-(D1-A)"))
 (segment (start 162.3 88) (end 157.774207 92.525793) (width 0.64) (layer "B.Cu") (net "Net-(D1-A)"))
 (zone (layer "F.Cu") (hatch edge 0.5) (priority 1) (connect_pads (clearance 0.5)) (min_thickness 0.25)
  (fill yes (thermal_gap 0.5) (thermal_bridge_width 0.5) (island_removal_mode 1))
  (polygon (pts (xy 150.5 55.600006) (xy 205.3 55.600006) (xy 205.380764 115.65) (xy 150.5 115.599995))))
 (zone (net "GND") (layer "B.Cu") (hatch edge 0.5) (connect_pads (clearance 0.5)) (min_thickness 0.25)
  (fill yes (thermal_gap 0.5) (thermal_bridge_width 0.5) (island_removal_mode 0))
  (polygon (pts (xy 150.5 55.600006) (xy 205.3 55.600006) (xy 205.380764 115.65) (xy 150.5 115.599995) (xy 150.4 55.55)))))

